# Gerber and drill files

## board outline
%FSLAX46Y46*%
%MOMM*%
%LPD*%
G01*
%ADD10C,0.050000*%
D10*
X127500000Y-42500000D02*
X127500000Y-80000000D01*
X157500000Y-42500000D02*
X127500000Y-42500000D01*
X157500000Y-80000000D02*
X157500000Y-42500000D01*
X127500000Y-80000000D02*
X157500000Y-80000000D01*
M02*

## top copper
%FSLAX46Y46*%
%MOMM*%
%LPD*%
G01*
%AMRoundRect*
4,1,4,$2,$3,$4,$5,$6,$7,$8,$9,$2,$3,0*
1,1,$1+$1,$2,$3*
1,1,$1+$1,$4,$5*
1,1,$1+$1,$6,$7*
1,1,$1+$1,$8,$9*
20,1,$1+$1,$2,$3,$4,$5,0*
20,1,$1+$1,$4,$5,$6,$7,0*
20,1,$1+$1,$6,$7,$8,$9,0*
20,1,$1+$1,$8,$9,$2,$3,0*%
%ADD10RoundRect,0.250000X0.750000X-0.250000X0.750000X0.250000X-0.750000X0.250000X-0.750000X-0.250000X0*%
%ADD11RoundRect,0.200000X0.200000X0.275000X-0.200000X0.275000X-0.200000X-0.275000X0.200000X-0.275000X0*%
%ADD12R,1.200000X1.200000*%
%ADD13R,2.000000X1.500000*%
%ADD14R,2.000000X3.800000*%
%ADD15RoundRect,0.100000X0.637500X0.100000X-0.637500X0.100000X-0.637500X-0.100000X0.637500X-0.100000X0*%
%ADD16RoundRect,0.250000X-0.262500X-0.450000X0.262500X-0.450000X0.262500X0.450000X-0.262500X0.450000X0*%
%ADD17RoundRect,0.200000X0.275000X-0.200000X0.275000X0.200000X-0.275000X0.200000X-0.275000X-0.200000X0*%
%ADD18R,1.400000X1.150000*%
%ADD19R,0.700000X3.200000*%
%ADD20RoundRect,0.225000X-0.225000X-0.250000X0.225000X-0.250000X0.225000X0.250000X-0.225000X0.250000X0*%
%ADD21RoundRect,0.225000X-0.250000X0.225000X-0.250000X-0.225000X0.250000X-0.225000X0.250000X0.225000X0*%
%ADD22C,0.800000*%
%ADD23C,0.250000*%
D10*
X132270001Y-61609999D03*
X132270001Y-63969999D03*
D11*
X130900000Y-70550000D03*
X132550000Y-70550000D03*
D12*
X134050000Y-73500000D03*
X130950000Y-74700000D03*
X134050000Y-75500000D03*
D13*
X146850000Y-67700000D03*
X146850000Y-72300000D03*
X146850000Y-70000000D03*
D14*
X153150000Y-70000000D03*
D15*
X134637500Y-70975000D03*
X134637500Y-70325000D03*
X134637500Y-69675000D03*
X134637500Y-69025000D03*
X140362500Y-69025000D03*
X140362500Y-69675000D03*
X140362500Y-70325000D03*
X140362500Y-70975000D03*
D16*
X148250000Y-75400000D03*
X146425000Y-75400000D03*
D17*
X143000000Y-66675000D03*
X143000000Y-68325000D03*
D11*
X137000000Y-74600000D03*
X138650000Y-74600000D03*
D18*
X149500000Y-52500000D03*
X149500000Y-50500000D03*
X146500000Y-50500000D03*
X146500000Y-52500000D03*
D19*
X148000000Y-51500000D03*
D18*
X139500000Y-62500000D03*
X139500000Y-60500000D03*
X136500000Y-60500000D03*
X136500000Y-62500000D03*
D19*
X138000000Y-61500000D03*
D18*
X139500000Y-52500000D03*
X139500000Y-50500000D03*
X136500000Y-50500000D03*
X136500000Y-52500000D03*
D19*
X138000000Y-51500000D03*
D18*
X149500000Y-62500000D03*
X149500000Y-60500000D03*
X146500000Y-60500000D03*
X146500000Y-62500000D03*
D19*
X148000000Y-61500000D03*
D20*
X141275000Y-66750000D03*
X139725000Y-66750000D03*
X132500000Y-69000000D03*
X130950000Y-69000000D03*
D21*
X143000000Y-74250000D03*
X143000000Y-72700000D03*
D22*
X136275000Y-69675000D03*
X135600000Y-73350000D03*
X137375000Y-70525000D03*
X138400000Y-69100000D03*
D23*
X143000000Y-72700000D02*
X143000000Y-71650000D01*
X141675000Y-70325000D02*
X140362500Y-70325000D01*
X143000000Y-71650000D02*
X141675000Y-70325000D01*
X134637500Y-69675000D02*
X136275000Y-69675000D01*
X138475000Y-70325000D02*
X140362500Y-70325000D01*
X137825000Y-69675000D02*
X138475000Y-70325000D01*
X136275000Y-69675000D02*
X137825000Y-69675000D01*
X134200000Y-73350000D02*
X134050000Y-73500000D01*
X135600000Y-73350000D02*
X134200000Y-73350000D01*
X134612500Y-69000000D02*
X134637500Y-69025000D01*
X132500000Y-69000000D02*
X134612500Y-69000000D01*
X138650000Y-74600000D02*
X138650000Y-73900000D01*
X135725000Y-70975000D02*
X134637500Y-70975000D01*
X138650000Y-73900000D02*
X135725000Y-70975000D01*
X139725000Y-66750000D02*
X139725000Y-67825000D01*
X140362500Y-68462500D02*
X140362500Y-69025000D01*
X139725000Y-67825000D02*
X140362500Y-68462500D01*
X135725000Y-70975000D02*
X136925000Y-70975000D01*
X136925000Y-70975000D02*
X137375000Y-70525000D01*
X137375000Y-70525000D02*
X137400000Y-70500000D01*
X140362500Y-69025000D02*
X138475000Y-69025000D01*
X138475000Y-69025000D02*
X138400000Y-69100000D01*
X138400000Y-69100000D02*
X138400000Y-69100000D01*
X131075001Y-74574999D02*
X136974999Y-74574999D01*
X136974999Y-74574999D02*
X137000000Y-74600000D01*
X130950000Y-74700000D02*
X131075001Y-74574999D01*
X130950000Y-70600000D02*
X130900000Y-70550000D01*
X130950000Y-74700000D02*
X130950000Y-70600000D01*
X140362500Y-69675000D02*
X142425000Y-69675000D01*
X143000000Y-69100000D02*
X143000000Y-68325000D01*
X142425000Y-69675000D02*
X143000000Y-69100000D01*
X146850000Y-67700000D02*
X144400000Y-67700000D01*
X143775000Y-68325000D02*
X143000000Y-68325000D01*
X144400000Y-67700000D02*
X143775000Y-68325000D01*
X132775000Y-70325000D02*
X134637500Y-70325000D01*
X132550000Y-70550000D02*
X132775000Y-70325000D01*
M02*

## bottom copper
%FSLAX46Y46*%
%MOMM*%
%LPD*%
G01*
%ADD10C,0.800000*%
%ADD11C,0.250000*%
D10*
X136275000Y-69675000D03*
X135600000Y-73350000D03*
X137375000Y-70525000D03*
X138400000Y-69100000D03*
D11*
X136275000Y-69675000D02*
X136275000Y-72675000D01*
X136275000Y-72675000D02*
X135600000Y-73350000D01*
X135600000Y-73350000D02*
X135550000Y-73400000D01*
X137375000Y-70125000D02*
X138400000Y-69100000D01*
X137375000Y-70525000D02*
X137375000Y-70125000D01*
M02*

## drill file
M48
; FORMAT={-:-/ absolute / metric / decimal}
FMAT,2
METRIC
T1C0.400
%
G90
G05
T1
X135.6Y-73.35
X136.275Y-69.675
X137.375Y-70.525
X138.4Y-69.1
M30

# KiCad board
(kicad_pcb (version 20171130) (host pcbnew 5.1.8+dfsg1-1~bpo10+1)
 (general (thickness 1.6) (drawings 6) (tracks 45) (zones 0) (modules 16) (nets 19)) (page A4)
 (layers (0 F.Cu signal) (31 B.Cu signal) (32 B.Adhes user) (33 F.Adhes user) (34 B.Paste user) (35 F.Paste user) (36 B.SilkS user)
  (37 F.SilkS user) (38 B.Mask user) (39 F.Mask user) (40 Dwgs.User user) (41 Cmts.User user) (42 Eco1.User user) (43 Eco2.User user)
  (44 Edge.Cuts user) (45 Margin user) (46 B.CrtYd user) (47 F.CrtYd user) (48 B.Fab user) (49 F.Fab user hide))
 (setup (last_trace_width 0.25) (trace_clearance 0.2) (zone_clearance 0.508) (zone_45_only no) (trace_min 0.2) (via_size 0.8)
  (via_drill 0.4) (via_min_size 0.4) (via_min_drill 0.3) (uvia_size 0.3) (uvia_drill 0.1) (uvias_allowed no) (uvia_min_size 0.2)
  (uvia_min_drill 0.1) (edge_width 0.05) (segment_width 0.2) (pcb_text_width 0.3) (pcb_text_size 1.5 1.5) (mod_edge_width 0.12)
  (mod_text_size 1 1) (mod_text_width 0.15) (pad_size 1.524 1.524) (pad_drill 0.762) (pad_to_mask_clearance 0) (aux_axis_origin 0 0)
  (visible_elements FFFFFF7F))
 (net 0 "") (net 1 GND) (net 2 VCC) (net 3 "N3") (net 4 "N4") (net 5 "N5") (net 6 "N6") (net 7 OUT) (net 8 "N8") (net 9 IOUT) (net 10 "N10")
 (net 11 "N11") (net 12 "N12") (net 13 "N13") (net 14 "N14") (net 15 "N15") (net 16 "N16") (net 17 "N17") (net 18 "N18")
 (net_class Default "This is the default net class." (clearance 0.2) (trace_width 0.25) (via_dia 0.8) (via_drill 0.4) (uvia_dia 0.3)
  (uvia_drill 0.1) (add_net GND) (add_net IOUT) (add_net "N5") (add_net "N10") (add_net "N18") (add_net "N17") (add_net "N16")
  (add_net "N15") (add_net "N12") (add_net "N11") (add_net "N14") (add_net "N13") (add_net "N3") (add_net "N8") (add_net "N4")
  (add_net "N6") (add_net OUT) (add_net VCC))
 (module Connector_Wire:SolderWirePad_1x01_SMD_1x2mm (layer F.Cu) (at 132.270001 61.609999 90)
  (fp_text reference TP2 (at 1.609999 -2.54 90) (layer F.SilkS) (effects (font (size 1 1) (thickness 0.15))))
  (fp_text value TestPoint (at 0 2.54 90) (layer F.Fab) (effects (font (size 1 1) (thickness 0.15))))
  (pad 1 smd roundrect (at 0 0 90) (size 1 2) (layers F.Cu F.Paste F.Mask) (roundrect_rratio 0.25) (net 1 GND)))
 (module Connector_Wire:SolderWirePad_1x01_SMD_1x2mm (layer F.Cu) (at 132.270001 63.969999 90)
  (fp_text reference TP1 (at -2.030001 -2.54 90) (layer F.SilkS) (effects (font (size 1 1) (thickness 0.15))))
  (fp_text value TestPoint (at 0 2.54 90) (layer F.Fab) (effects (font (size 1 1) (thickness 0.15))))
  (pad 1 smd roundrect (at 0 0 90) (size 1 2) (layers F.Cu F.Paste F.Mask) (roundrect_rratio 0.25) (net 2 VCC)))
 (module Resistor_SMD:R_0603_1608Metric (layer F.Cu) (at 131.725 70.55 180)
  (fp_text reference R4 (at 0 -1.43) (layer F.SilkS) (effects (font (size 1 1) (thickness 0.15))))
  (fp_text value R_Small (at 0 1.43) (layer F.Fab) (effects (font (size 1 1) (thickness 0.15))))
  (pad 2 smd roundrect (at 0.825 0 180) (size 0.8 0.95) (layers F.Cu F.Paste F.Mask) (roundrect_rratio 0.25) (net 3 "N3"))
  (pad 1 smd roundrect (at -0.825 0 180) (size 0.8 0.95) (layers F.Cu F.Paste F.Mask) (roundrect_rratio 0.25) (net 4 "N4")))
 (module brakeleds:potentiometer (layer F.Cu) (at 132.75 74.6 180)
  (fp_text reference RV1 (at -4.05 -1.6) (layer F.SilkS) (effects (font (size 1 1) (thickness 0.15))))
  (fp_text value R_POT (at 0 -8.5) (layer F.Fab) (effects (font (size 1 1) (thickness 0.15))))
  (pad 3 smd rect (at -1.3 1.1 270) (size 1.2 1.2) (layers F.Cu F.Paste F.Mask) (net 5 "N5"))
  (pad 2 smd rect (at 1.8 -0.1 270) (size 1.2 1.2) (layers F.Cu F.Paste F.Mask) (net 3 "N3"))
  (pad 1 smd rect (at -1.3 -0.9 270) (size 1.2 1.2) (layers F.Cu F.Paste F.Mask) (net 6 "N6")))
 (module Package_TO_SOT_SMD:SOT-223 (layer F.Cu) (at 150 70)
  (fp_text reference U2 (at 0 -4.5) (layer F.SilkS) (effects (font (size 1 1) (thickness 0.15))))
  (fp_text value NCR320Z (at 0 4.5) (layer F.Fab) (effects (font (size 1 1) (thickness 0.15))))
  (pad 1 smd rect (at -3.15 -2.3) (size 2 1.5) (layers F.Cu F.Paste F.Mask) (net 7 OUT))
  (pad 3 smd rect (at -3.15 2.3) (size 2 1.5) (layers F.Cu F.Paste F.Mask) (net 1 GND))
  (pad 2 smd rect (at -3.15 0) (size 2 1.5) (layers F.Cu F.Paste F.Mask) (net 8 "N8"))
  (pad 4 smd rect (at 3.15 0) (size 2 3.8) (layers F.Cu F.Paste F.Mask) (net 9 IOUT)))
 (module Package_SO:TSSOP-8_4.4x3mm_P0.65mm (layer F.Cu) (at 137.5 70 180)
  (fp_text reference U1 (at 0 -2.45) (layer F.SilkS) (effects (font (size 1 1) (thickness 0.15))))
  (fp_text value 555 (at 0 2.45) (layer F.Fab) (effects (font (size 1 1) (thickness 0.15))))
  (pad 8 smd roundrect (at 2.8625 -0.975 180) (size 1.475 0.4) (layers F.Cu F.Paste F.Mask) (roundrect_rratio 0.25) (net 2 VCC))
  (pad 7 smd roundrect (at 2.8625 -0.325 180) (size 1.475 0.4) (layers F.Cu F.Paste F.Mask) (roundrect_rratio 0.25) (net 4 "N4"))
  (pad 6 smd roundrect (at 2.8625 0.325 180) (size 1.475 0.4) (layers F.Cu F.Paste F.Mask) (roundrect_rratio 0.25) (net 5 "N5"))
  (pad 5 smd roundrect (at 2.8625 0.975 180) (size 1.475 0.4) (layers F.Cu F.Paste F.Mask) (roundrect_rratio 0.25) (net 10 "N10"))
  (pad 4 smd roundrect (at -2.8625 0.975 180) (size 1.475 0.4) (layers F.Cu F.Paste F.Mask) (roundrect_rratio 0.25) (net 2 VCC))
  (pad 3 smd roundrect (at -2.8625 0.325 180) (size 1.475 0.4) (layers F.Cu F.Paste F.Mask) (roundrect_rratio 0.25) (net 7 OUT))
  (pad 2 smd roundrect (at -2.8625 -0.325 180) (size 1.475 0.4) (layers F.Cu F.Paste F.Mask) (roundrect_rratio 0.25) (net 5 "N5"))
  (pad 1 smd roundrect (at -2.8625 -0.975 180) (size 1.475 0.4) (layers F.Cu F.Paste F.Mask) (roundrect_rratio 0.25) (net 1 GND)))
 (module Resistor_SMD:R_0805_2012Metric (layer F.Cu) (at 147.3375 75.4)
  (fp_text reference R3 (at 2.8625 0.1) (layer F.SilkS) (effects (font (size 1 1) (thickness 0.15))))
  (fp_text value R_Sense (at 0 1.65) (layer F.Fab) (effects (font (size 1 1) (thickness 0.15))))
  (pad 2 smd roundrect (at 0.9125 0) (size 1.025 1.4) (layers F.Cu F.Paste F.Mask) (roundrect_rratio 0.243902) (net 8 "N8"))
  (pad 1 smd roundrect (at -0.9125 0) (size 1.025 1.4) (layers F.Cu F.Paste F.Mask) (roundrect_rratio 0.243902) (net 1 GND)))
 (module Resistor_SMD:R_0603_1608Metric (layer F.Cu) (at 143 67.5 90)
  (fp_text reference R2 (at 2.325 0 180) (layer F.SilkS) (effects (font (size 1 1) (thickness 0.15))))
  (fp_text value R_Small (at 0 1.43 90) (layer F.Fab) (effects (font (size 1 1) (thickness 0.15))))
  (pad 2 smd roundrect (at 0.825 0 90) (size 0.8 0.95) (layers F.Cu F.Paste F.Mask) (roundrect_rratio 0.25) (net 1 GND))
  (pad 1 smd roundrect (at -0.825 0 90) (size 0.8 0.95) (layers F.Cu F.Paste F.Mask) (roundrect_rratio 0.25) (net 7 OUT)))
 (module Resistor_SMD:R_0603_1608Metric (layer F.Cu) (at 137.825 74.6 180)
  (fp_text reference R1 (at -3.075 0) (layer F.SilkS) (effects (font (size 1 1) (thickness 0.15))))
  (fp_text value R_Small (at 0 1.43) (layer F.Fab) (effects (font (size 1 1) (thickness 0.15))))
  (pad 2 smd roundrect (at 0.825 0 180) (size 0.8 0.95) (layers F.Cu F.Paste F.Mask) (roundrect_rratio 0.25) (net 3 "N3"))
  (pad 1 smd roundrect (at -0.825 0 180) (size 0.8 0.95) (layers F.Cu F.Paste F.Mask) (roundrect_rratio 0.25) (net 2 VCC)))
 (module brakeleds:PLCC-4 (layer F.Cu) (at 148 51.5)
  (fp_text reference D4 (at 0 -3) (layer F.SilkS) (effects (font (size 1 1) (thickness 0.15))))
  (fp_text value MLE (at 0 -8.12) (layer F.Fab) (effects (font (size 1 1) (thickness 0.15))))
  (pad 2 smd rect (at 1.5 1) (size 1.4 1.15) (layers F.Cu F.Paste F.Mask) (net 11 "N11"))
  (pad 1 smd rect (at 1.5 -1) (size 1.4 1.15) (layers F.Cu F.Paste F.Mask) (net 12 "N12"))
  (pad 4 smd rect (at -1.5 -1) (size 1.4 1.15) (layers F.Cu F.Paste F.Mask) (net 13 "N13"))
  (pad 3 smd rect (at -1.5 1) (size 1.4 1.15) (layers F.Cu F.Paste F.Mask) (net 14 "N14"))
  (pad 5 smd rect (at 0 0) (size 0.7 3.2) (layers F.Cu F.Paste F.Mask) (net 1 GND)))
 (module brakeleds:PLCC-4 (layer F.Cu) (at 138 61.5)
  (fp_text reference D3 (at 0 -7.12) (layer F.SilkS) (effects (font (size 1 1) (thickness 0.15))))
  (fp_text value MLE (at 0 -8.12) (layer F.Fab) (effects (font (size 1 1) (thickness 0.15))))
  (pad 2 smd rect (at 1.5 1) (size 1.4 1.15) (layers F.Cu F.Paste F.Mask) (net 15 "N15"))
  (pad 1 smd rect (at 1.5 -1) (size 1.4 1.15) (layers F.Cu F.Paste F.Mask) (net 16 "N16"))
  (pad 4 smd rect (at -1.5 -1) (size 1.4 1.15) (layers F.Cu F.Paste F.Mask) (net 11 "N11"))
  (pad 3 smd rect (at -1.5 1) (size 1.4 1.15) (layers F.Cu F.Paste F.Mask) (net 12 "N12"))
  (pad 5 smd rect (at 0 0) (size 0.7 3.2) (layers F.Cu F.Paste F.Mask) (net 1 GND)))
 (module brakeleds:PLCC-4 (layer F.Cu) (at 138 51.5)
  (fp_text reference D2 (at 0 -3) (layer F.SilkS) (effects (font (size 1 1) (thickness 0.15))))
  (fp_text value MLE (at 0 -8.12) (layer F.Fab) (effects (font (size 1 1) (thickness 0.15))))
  (pad 2 smd rect (at 1.5 1) (size 1.4 1.15) (layers F.Cu F.Paste F.Mask) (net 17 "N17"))
  (pad 1 smd rect (at 1.5 -1) (size 1.4 1.15) (layers F.Cu F.Paste F.Mask) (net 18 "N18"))
  (pad 4 smd rect (at -1.5 -1) (size 1.4 1.15) (layers F.Cu F.Paste F.Mask) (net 15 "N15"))
  (pad 3 smd rect (at -1.5 1) (size 1.4 1.15) (layers F.Cu F.Paste F.Mask) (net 16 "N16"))
  (pad 5 smd rect (at 0 0) (size 0.7 3.2) (layers F.Cu F.Paste F.Mask) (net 1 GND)))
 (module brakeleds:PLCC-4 (layer F.Cu) (at 148 61.5)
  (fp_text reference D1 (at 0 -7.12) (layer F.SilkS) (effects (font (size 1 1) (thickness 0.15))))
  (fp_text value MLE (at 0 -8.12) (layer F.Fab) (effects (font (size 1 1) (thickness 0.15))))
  (pad 2 smd rect (at 1.5 1) (size 1.4 1.15) (layers F.Cu F.Paste F.Mask) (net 9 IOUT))
  (pad 1 smd rect (at 1.5 -1) (size 1.4 1.15) (layers F.Cu F.Paste F.Mask) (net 9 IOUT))
  (pad 4 smd rect (at -1.5 -1) (size 1.4 1.15) (layers F.Cu F.Paste F.Mask) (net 17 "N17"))
  (pad 3 smd rect (at -1.5 1) (size 1.4 1.15) (layers F.Cu F.Paste F.Mask) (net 18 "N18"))
  (pad 5 smd rect (at 0 0) (size 0.7 3.2) (layers F.Cu F.Paste F.Mask) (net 1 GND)))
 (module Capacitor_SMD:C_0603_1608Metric (layer F.Cu) (at 140.5 66.75)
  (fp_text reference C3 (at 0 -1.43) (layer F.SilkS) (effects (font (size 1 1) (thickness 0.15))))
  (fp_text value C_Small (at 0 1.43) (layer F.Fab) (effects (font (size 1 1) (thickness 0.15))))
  (pad 2 smd roundrect (at 0.775 0) (size 0.9 0.95) (layers F.Cu F.Paste F.Mask) (roundrect_rratio 0.25) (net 1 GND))
  (pad 1 smd roundrect (at -0.775 0) (size 0.9 0.95) (layers F.Cu F.Paste F.Mask) (roundrect_rratio 0.25) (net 2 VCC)))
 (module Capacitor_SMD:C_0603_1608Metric (layer F.Cu) (at 131.725 69)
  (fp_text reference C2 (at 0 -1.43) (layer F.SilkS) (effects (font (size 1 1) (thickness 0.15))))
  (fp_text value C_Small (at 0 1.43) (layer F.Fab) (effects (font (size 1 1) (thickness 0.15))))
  (pad 2 smd roundrect (at 0.775 0) (size 0.9 0.95) (layers F.Cu F.Paste F.Mask) (roundrect_rratio 0.25) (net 10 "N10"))
  (pad 1 smd roundrect (at -0.775 0) (size 0.9 0.95) (layers F.Cu F.Paste F.Mask) (roundrect_rratio 0.25) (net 1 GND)))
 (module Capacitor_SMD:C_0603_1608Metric (layer F.Cu) (at 143 73.475 270)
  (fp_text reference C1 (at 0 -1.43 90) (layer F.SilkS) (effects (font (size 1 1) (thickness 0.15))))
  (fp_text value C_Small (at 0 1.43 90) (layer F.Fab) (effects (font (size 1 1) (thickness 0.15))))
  (pad 2 smd roundrect (at 0.775 0 270) (size 0.9 0.95) (layers F.Cu F.Paste F.Mask) (roundrect_rratio 0.25) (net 1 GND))
  (pad 1 smd roundrect (at -0.775 0 270) (size 0.9 0.95) (layers F.Cu F.Paste F.Mask) (roundrect_rratio 0.25) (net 5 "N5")))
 (gr_line (start 127.5 42.5) (end 127.5 80) (layer Edge.Cuts) (width 0.05))
 (gr_line (start 157.5 42.5) (end 127.5 42.5) (layer Edge.Cuts) (width 0.05))
 (gr_line (start 157.5 80) (end 157.5 42.5) (layer Edge.Cuts) (width 0.05))
 (gr_line (start 127.5 80) (end 157.5 80) (layer Edge.Cuts) (width 0.05))
 (segment (start 143 72.7) (end 143 71.65) (width 0.25) (layer F.Cu) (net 5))
 (segment (start 141.675 70.325) (end 140.3625 70.325) (width 0.25) (layer F.Cu) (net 5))
 (segment (start 143 71.65) (end 141.675 70.325) (width 0.25) (layer F.Cu) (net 5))
 (segment (start 134.6375 69.675) (end 136.275 69.675) (width 0.25) (layer F.Cu) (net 5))
 (segment (start 138.475 70.325) (end 140.3625 70.325) (width 0.25) (layer F.Cu) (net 5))
 (segment (start 137.825 69.675) (end 138.475 70.325) (width 0.25) (layer F.Cu) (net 5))
 (segment (start 136.275 69.675) (end 137.825 69.675) (width 0.25) (layer F.Cu) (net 5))
 (via (at 136.275 69.675) (size 0.8) (drill 0.4) (layers F.Cu B.Cu) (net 5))
 (segment (start 136.275 69.675) (end 136.275 72.675) (width 0.25) (layer B.Cu) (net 5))
 (segment (start 136.275 72.675) (end 135.6 73.35) (width 0.25) (layer B.Cu) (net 5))
 (segment (start 135.6 73.35) (end 135.55 73.4) (width 0.25) (layer B.Cu) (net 5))
 (via (at 135.6 73.35) (size 0.8) (drill 0.4) (layers F.Cu B.Cu) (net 5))
 (segment (start 134.2 73.35) (end 134.05 73.5) (width 0.25) (layer F.Cu) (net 5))
 (segment (start 135.6 73.35) (end 134.2 73.35) (width 0.25) (layer F.Cu) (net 5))
 (segment (start 134.6125 69) (end 134.6375 69.025) (width 0.25) (layer F.Cu) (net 10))
 (segment (start 132.5 69) (end 134.6125 69) (width 0.25) (layer F.Cu) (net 10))
 (segment (start 138.65 74.6) (end 138.65 73.9) (width 0.25) (layer F.Cu) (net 2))
 (segment (start 135.725 70.975) (end 134.6375 70.975) (width 0.25) (layer F.Cu) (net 2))
 (segment (start 138.65 73.9) (end 135.725 70.975) (width 0.25) (layer F.Cu) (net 2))
 (segment (start 139.725 66.75) (end 139.725 67.825) (width 0.25) (layer F.Cu) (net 2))
 (segment (start 140.3625 68.4625) (end 140.3625 69.025) (width 0.25) (layer F.Cu) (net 2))
 (segment (start 139.725 67.825) (end 140.3625 68.4625) (width 0.25) (layer F.Cu) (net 2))
 (segment (start 135.725 70.975) (end 136.925 70.975) (width 0.25) (layer F.Cu) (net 2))
 (segment (start 136.925 70.975) (end 137.375 70.525) (width 0.25) (layer F.Cu) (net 2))
 (segment (start 137.375 70.525) (end 137.4 70.5) (width 0.25) (layer F.Cu) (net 2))
 (via (at 137.375 70.525) (size 0.8) (drill 0.4) (layers F.Cu B.Cu) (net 2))
 (segment (start 140.3625 69.025) (end 138.475 69.025) (width 0.25) (layer F.Cu) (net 2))
 (segment (start 138.475 69.025) (end 138.4 69.1) (width 0.25) (layer F.Cu) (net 2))
 (segment (start 138.4 69.1) (end 138.4 69.1) (width 0.25) (layer F.Cu) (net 2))
 (via (at 138.4 69.1) (size 0.8) (drill 0.4) (layers F.Cu B.Cu) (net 2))
 (segment (start 137.375 70.125) (end 138.4 69.1) (width 0.25) (layer B.Cu) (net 2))
 (segment (start 137.375 70.525) (end 137.375 70.125) (width 0.25) (layer B.Cu) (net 2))
 (segment (start 131.075001 74.574999) (end 136.974999 74.574999) (width 0.25) (layer F.Cu) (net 3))
 (segment (start 136.974999 74.574999) (end 137 74.6) (width 0.25) (layer F.Cu) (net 3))
 (segment (start 130.95 74.7) (end 131.075001 74.574999) (width 0.25) (layer F.Cu) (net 3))
 (segment (start 130.95 70.6) (end 130.9 70.55) (width 0.25) (layer F.Cu) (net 3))
 (segment (start 130.95 74.7) (end 130.95 70.6) (width 0.25) (layer F.Cu) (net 3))
 (segment (start 140.3625 69.675) (end 142.425 69.675) (width 0.25) (layer F.Cu) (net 7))
 (segment (start 143 69.1) (end 143 68.325) (width 0.25) (layer F.Cu) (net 7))
 (segment (start 142.425 69.675) (end 143 69.1) (width 0.25) (layer F.Cu) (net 7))
 (segment (start 146.85 67.7) (end 144.4 67.7) (width 0.25) (layer F.Cu) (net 7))
 (segment (start 143.775 68.325) (end 143 68.325) (width 0.25) (layer F.Cu) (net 7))
 (segment (start 144.4 67.7) (end 143.775 68.325) (width 0.25) (layer F.Cu) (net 7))
 (segment (start 132.775 70.325) (end 134.6375 70.325) (width 0.25) (layer F.Cu) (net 4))
 (segment (start 132.55 70.55) (end 132.775 70.325) (width 0.25) (layer F.Cu) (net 4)))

